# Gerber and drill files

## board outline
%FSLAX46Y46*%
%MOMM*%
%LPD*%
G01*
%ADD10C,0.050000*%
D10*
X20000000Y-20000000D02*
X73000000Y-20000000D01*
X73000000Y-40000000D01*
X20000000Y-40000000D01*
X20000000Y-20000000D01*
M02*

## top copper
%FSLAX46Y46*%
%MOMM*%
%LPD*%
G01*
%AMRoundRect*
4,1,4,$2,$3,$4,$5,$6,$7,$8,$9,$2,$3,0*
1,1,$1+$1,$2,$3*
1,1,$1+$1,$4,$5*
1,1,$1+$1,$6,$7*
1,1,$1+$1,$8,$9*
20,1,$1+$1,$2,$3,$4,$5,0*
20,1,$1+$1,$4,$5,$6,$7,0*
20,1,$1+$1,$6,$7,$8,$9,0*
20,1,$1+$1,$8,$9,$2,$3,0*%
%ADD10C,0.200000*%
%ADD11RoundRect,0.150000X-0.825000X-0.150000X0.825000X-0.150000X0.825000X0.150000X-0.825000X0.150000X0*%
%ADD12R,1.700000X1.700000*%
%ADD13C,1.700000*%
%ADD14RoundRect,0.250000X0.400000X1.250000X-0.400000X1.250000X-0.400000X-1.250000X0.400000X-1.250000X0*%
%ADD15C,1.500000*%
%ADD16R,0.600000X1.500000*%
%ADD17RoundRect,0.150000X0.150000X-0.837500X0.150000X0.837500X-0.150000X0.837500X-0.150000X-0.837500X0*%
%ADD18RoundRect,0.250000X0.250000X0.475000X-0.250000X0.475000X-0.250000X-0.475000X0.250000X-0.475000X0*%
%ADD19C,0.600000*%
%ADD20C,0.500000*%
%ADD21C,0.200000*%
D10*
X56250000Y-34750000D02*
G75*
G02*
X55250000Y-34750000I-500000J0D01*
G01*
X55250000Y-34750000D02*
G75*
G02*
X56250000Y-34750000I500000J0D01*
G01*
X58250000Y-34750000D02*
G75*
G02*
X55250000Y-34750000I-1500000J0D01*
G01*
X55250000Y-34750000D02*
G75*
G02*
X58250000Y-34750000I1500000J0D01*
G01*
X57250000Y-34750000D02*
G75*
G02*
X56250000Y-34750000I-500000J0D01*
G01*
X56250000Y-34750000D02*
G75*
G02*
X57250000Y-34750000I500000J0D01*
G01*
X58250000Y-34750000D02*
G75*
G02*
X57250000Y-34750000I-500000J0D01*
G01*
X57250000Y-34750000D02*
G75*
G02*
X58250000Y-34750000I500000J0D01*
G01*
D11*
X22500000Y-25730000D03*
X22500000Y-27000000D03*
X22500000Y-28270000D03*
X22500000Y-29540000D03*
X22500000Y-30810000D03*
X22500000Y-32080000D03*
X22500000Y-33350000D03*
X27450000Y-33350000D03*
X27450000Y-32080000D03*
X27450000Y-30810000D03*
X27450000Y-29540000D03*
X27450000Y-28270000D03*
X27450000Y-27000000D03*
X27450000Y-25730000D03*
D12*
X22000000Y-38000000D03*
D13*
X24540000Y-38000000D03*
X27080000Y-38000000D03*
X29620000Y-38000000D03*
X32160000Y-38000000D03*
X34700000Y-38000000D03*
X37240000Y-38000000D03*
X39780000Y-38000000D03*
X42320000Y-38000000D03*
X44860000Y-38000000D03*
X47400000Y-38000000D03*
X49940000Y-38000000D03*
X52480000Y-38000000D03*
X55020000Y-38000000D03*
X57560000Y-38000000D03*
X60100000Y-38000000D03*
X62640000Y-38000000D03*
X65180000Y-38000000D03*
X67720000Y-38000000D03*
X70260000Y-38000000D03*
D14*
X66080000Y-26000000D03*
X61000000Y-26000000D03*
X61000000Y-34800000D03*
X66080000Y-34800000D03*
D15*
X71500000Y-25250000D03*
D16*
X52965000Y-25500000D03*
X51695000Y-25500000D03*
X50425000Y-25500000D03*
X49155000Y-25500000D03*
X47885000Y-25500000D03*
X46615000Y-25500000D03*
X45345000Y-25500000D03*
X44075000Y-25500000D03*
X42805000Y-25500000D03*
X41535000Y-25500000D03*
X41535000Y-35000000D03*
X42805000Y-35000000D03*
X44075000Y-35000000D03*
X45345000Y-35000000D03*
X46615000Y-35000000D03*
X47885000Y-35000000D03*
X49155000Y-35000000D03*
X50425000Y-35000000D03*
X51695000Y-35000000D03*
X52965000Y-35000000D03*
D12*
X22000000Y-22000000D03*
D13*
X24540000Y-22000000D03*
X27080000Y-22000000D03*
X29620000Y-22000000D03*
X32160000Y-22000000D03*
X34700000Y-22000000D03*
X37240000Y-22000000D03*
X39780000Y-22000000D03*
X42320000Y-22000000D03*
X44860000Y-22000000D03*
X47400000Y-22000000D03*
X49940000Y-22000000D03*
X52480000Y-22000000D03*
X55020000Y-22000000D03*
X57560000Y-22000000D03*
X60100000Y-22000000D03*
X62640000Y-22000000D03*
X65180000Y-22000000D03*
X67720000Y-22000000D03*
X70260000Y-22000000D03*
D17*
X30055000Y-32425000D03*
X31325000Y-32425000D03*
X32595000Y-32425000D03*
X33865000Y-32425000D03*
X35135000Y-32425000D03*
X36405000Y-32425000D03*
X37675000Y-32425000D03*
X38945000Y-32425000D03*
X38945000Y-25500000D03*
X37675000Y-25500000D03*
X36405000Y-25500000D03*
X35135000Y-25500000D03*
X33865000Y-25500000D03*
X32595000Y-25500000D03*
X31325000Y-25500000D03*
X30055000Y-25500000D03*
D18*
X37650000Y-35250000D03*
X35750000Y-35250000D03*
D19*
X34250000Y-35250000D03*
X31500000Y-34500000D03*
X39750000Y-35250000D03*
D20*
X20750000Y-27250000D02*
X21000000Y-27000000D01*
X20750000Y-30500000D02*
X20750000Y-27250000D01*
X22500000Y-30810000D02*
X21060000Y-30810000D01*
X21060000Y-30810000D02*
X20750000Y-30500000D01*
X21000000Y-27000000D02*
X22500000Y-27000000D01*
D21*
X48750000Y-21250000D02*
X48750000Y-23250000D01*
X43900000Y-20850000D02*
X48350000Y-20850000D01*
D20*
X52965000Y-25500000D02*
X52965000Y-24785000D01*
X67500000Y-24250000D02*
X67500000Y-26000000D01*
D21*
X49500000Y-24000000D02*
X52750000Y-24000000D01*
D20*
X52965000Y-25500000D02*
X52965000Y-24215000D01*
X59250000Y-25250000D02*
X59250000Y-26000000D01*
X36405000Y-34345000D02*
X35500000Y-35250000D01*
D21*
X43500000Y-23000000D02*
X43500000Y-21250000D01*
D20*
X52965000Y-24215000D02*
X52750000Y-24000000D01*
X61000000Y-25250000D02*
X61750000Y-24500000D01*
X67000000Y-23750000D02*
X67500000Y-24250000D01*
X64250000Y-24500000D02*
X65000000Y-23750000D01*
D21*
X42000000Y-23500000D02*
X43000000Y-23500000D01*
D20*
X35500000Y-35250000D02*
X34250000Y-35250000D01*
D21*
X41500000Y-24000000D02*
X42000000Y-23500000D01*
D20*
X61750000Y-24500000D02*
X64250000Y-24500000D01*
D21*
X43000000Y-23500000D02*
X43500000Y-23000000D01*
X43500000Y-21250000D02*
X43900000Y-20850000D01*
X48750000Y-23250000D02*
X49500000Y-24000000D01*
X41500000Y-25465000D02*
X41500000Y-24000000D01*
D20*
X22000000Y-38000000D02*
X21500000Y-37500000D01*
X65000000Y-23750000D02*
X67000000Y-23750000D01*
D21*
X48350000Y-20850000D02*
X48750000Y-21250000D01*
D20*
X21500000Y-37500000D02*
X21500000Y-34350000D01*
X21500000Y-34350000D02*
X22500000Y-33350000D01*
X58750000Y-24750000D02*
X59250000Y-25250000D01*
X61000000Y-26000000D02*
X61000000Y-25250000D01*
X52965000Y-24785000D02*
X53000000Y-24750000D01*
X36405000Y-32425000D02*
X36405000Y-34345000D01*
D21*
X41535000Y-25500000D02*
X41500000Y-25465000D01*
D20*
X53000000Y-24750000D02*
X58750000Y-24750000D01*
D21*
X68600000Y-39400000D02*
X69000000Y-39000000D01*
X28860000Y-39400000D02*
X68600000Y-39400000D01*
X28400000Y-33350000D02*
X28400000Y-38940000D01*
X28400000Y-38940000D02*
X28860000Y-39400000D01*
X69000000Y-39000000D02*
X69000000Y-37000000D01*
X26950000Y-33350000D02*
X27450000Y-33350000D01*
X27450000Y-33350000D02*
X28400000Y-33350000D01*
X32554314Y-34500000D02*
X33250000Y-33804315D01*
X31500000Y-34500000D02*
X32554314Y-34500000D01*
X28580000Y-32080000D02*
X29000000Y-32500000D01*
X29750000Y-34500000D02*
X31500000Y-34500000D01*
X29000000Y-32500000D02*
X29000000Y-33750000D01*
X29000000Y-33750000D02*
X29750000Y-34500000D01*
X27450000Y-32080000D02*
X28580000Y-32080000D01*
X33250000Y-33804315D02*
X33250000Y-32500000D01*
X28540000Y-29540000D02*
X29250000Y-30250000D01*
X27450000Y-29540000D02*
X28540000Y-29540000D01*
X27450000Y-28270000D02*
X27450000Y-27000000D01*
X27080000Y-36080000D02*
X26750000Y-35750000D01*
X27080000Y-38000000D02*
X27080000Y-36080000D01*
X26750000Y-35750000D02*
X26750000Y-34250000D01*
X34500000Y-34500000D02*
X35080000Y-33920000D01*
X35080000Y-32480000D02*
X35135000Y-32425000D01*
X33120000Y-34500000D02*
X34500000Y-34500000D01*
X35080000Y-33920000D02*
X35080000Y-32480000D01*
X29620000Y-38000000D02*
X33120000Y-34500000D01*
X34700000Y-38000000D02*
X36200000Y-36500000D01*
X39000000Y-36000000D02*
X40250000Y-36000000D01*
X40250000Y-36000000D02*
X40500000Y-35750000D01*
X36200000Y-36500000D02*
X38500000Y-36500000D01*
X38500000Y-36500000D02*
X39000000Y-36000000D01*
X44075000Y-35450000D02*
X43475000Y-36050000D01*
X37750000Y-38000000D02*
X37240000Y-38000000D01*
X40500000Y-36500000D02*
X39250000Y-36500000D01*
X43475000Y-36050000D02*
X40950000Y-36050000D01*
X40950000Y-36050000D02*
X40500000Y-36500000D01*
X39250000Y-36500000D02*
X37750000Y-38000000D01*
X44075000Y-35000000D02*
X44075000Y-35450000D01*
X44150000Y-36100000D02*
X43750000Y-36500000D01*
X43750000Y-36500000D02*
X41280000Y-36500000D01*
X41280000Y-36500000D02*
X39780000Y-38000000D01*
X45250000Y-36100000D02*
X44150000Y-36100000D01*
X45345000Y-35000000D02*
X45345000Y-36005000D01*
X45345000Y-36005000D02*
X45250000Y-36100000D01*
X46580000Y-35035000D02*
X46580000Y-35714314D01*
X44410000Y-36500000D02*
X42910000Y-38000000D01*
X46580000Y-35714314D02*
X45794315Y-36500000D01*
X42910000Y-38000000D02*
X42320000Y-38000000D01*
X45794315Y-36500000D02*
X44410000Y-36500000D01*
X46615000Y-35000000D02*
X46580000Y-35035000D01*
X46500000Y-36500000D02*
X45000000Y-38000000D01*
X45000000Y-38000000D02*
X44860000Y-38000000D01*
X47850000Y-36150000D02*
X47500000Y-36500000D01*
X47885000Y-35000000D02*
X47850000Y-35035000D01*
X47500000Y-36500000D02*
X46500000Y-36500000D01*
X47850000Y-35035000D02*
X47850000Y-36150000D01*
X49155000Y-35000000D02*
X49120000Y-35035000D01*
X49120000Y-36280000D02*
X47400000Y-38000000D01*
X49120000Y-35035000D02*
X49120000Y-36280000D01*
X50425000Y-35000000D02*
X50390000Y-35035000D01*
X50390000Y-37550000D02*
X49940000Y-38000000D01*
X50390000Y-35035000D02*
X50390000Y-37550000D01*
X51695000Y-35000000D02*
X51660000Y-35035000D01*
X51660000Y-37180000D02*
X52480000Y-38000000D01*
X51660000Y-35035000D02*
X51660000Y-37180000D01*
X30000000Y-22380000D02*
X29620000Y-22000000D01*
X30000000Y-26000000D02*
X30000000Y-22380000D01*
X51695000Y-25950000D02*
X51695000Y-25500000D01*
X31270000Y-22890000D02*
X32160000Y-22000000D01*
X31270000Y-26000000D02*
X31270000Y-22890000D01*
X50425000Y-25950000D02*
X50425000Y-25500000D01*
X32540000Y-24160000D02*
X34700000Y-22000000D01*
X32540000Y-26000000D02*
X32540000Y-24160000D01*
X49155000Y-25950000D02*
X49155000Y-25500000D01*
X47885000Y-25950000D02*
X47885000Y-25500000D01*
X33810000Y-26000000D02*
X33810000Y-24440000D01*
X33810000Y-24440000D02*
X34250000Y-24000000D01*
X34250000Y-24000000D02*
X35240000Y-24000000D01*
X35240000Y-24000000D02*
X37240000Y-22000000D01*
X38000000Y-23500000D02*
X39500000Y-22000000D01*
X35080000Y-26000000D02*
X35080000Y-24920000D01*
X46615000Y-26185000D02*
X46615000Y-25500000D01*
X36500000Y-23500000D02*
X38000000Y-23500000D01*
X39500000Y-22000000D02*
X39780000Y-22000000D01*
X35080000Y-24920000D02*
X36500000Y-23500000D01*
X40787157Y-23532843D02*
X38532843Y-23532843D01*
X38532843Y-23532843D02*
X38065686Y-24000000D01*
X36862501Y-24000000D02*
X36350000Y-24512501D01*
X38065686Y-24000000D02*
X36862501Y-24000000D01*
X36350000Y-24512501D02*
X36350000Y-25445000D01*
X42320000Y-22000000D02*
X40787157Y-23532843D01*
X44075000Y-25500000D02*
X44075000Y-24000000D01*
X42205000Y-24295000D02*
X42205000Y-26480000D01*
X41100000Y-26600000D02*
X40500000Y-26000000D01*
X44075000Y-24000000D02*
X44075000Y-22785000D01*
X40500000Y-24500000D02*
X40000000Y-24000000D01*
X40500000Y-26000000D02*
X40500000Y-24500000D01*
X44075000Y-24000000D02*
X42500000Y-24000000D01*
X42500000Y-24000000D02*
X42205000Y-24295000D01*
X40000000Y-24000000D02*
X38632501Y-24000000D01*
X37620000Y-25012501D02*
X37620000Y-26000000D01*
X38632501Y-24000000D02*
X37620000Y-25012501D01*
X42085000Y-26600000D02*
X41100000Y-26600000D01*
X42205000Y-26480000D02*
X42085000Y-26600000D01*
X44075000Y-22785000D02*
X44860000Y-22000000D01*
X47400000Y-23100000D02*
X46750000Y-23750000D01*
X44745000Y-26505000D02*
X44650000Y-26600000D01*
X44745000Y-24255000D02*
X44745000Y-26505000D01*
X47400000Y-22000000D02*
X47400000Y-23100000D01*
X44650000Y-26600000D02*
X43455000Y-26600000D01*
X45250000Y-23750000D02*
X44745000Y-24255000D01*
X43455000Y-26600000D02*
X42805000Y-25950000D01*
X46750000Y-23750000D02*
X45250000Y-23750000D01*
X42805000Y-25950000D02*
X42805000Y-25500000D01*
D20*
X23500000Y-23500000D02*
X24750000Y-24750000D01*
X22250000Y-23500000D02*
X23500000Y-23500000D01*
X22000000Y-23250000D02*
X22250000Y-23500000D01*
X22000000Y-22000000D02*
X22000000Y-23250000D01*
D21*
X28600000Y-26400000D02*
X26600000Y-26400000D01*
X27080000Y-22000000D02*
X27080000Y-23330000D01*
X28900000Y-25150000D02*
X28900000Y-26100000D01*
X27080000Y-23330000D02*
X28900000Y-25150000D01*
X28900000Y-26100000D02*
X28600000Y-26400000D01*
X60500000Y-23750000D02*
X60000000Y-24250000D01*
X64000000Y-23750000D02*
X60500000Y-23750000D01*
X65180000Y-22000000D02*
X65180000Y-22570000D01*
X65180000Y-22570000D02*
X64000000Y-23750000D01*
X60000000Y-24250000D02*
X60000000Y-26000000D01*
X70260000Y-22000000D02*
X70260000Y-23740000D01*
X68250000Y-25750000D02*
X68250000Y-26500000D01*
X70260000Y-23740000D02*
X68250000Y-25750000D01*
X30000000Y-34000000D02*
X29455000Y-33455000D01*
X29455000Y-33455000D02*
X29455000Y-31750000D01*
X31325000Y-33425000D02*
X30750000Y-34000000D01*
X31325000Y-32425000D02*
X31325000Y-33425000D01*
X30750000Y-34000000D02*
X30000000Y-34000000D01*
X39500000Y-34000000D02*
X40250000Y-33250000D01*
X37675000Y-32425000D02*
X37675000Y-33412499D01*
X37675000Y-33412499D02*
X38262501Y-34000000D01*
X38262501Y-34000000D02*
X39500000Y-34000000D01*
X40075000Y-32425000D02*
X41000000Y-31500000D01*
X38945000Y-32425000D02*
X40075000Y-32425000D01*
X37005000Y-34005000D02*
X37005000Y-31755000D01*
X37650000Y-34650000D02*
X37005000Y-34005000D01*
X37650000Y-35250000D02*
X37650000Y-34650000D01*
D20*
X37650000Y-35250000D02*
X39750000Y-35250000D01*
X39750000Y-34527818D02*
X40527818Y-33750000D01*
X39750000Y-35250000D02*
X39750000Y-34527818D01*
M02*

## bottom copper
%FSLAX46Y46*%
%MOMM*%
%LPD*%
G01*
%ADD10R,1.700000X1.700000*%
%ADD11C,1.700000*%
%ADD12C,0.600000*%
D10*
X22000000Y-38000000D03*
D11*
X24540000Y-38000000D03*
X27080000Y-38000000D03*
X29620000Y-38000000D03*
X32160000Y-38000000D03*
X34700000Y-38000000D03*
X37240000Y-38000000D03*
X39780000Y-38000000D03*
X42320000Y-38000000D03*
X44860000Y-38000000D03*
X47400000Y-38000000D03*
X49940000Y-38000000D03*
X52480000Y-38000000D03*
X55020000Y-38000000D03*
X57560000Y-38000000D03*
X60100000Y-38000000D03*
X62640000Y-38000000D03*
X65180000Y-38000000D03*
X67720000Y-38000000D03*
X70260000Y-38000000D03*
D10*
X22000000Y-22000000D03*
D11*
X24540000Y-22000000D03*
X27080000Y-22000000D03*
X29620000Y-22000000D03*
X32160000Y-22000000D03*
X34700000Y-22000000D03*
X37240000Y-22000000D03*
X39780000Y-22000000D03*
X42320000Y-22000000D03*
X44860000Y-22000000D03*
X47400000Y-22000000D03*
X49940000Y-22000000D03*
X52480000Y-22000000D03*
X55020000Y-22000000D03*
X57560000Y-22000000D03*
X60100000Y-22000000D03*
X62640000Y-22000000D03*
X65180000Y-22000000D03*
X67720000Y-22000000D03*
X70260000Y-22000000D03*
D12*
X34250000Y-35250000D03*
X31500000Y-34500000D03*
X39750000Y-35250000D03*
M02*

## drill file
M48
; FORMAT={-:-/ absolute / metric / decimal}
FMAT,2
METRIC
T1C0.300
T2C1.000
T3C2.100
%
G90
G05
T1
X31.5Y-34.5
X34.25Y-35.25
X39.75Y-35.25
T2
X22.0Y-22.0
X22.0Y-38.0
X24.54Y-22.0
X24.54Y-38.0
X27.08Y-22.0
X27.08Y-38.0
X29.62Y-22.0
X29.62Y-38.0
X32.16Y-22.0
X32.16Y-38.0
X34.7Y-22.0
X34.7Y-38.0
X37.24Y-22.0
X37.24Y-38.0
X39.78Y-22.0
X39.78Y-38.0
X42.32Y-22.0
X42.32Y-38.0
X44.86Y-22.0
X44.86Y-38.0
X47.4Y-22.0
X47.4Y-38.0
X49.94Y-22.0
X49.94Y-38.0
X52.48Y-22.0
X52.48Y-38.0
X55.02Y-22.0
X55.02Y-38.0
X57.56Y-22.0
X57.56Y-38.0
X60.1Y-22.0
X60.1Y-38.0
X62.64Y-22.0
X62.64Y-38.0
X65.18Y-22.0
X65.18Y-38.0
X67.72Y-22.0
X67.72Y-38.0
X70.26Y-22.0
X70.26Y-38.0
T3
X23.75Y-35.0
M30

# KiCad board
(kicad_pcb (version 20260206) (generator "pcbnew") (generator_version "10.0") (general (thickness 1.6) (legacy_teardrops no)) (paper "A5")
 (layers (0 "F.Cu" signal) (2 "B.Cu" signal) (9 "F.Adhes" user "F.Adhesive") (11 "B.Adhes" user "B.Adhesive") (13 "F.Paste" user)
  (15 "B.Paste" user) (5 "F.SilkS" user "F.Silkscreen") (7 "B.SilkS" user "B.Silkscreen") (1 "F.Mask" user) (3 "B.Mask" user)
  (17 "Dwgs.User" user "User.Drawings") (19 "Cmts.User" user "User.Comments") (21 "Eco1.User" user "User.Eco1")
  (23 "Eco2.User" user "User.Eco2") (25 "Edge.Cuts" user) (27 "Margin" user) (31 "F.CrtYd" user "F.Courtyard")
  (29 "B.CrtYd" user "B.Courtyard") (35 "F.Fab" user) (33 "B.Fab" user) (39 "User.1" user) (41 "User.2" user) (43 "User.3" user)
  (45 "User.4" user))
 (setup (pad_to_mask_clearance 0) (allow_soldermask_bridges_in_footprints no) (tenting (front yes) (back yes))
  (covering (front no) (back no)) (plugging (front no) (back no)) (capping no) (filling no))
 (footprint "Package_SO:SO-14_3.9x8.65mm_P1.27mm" (layer "F.Cu") (at 24.975 29.54)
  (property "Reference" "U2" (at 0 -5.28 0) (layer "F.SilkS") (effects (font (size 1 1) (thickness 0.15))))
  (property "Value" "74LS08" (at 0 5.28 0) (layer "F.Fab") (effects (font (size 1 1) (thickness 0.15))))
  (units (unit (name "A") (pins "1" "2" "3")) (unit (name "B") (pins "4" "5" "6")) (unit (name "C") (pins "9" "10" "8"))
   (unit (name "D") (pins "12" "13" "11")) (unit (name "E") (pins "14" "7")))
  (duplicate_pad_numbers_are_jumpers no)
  (pad "1" smd roundrect (at -2.475 -3.81) (size 1.95 0.6) (layers "F.Cu" "F.Mask" "F.Paste") (roundrect_rratio 0.25)
   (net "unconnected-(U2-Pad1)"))
  (pad "2" smd roundrect (at -2.475 -2.54) (size 1.95 0.6) (layers "F.Cu" "F.Mask" "F.Paste") (roundrect_rratio 0.25) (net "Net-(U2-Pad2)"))
  (pad "3" smd roundrect (at -2.475 -1.27) (size 1.95 0.6) (layers "F.Cu" "F.Mask" "F.Paste") (roundrect_rratio 0.25)
   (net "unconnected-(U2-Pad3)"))
  (pad "4" smd roundrect (at -2.475 0) (size 1.95 0.6) (layers "F.Cu" "F.Mask" "F.Paste") (roundrect_rratio 0.25)
   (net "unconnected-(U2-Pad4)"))
  (pad "5" smd roundrect (at -2.475 1.27) (size 1.95 0.6) (layers "F.Cu" "F.Mask" "F.Paste") (roundrect_rratio 0.25) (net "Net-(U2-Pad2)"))
  (pad "6" smd roundrect (at -2.475 2.54) (size 1.95 0.6) (layers "F.Cu" "F.Mask" "F.Paste") (roundrect_rratio 0.25)
   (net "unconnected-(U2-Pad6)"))
  (pad "7" smd roundrect (at -2.475 3.81) (size 1.95 0.6) (layers "F.Cu" "F.Mask" "F.Paste") (roundrect_rratio 0.25) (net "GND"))
  (pad "8" smd roundrect (at 2.475 3.81) (size 1.95 0.6) (layers "F.Cu" "F.Mask" "F.Paste") (roundrect_rratio 0.25)
   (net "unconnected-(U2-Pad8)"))
  (pad "9" smd roundrect (at 2.475 2.54) (size 1.95 0.6) (layers "F.Cu" "F.Mask" "F.Paste") (roundrect_rratio 0.25)
   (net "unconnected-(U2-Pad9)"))
  (pad "10" smd roundrect (at 2.475 1.27) (size 1.95 0.6) (layers "F.Cu" "F.Mask" "F.Paste") (roundrect_rratio 0.25)
   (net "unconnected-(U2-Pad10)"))
  (pad "11" smd roundrect (at 2.475 0) (size 1.95 0.6) (layers "F.Cu" "F.Mask" "F.Paste") (roundrect_rratio 0.25)
   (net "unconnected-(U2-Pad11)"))
  (pad "12" smd roundrect (at 2.475 -1.27) (size 1.95 0.6) (layers "F.Cu" "F.Mask" "F.Paste") (roundrect_rratio 0.25) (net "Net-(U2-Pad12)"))
  (pad "13" smd roundrect (at 2.475 -2.54) (size 1.95 0.6) (layers "F.Cu" "F.Mask" "F.Paste") (roundrect_rratio 0.25) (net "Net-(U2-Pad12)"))
  (pad "14" smd roundrect (at 2.475 -3.81) (size 1.95 0.6) (layers "F.Cu" "F.Mask" "F.Paste") (roundrect_rratio 0.25)
   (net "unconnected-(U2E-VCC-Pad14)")))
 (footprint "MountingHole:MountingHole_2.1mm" (layer "F.Cu") (at 23.75 35)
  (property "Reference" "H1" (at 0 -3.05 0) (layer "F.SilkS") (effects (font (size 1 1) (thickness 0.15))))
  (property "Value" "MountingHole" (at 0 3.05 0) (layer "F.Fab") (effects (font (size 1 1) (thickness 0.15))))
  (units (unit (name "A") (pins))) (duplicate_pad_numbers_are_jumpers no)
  (pad "" np_thru_hole circle (at 0 0) (size 2.1 2.1) (drill 2.1) (layers "*.Cu" "*.Mask")))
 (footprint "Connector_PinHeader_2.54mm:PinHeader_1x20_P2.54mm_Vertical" (layer "F.Cu") (at 22 38 90)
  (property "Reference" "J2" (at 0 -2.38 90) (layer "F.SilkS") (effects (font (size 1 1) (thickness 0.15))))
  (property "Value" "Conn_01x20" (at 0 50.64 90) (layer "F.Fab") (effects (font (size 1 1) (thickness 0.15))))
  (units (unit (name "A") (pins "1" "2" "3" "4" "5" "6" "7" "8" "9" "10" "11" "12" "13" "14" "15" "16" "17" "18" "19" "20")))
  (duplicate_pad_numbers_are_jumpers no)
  (pad "1" thru_hole rect (at 0 0 90) (size 1.7 1.7) (drill 1) (layers "*.Cu" "*.Mask") (remove_unused_layers no) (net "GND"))
  (pad "2" thru_hole circle (at 0 2.54 90) (size 1.7 1.7) (drill 1) (layers "*.Cu" "*.Mask") (remove_unused_layers no)
   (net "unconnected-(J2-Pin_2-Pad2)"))
  (pad "3" thru_hole circle (at 0 5.08 90) (size 1.7 1.7) (drill 1) (layers "*.Cu" "*.Mask") (remove_unused_layers no)
   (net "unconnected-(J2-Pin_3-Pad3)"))
  (pad "4" thru_hole circle (at 0 7.62 90) (size 1.7 1.7) (drill 1) (layers "*.Cu" "*.Mask") (remove_unused_layers no) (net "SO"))
  (pad "5" thru_hole circle (at 0 10.16 90) (size 1.7 1.7) (drill 1) (layers "*.Cu" "*.Mask") (remove_unused_layers no)
   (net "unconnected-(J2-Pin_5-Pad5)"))
  (pad "6" thru_hole circle (at 0 12.7 90) (size 1.7 1.7) (drill 1) (layers "*.Cu" "*.Mask") (remove_unused_layers no)
   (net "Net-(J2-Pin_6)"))
  (pad "7" thru_hole circle (at 0 15.24 90) (size 1.7 1.7) (drill 1) (layers "*.Cu" "*.Mask") (remove_unused_layers no)
   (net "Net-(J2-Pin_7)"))
  (pad "8" thru_hole circle (at 0 17.78 90) (size 1.7 1.7) (drill 1) (layers "*.Cu" "*.Mask") (remove_unused_layers no)
   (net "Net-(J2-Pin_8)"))
  (pad "9" thru_hole circle (at 0 20.32 90) (size 1.7 1.7) (drill 1) (layers "*.Cu" "*.Mask") (remove_unused_layers no)
   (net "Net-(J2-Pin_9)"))
  (pad "10" thru_hole circle (at 0 22.86 90) (size 1.7 1.7) (drill 1) (layers "*.Cu" "*.Mask") (remove_unused_layers no)
   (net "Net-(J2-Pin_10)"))
  (pad "11" thru_hole circle (at 0 25.4 90) (size 1.7 1.7) (drill 1) (layers "*.Cu" "*.Mask") (remove_unused_layers no)
   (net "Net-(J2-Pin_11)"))
  (pad "12" thru_hole circle (at 0 27.94 90) (size 1.7 1.7) (drill 1) (layers "*.Cu" "*.Mask") (remove_unused_layers no)
   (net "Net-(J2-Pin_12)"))
  (pad "13" thru_hole circle (at 0 30.48 90) (size 1.7 1.7) (drill 1) (layers "*.Cu" "*.Mask") (remove_unused_layers no)
   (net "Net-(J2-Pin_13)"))
  (pad "14" thru_hole circle (at 0 33.02 90) (size 1.7 1.7) (drill 1) (layers "*.Cu" "*.Mask") (remove_unused_layers no)
   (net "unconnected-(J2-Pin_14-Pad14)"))
  (pad "15" thru_hole circle (at 0 35.56 90) (size 1.7 1.7) (drill 1) (layers "*.Cu" "*.Mask") (remove_unused_layers no)
   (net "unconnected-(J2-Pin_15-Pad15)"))
  (pad "16" thru_hole circle (at 0 38.1 90) (size 1.7 1.7) (drill 1) (layers "*.Cu" "*.Mask") (remove_unused_layers no)
   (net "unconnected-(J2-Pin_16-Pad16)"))
  (pad "17" thru_hole circle (at 0 40.64 90) (size 1.7 1.7) (drill 1) (layers "*.Cu" "*.Mask") (remove_unused_layers no)
   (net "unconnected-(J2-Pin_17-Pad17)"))
  (pad "18" thru_hole circle (at 0 43.18 90) (size 1.7 1.7) (drill 1) (layers "*.Cu" "*.Mask") (remove_unused_layers no)
   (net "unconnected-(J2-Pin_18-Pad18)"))
  (pad "19" thru_hole circle (at 0 45.72 90) (size 1.7 1.7) (drill 1) (layers "*.Cu" "*.Mask") (remove_unused_layers no)
   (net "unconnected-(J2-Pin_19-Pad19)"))
  (pad "20" thru_hole circle (at 0 48.26 90) (size 1.7 1.7) (drill 1) (layers "*.Cu" "*.Mask") (remove_unused_layers no)
   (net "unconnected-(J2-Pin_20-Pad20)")))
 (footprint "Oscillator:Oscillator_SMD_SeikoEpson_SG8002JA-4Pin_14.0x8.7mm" (layer "F.Cu") (at 63.54 30.4 180)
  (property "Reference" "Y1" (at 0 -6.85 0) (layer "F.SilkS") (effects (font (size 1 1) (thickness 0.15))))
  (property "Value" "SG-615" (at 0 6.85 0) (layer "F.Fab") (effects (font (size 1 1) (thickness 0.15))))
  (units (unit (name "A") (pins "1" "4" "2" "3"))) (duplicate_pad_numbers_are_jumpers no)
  (pad "1" smd roundrect (at -2.54 4.4 180) (size 1.3 3) (layers "F.Cu" "F.Mask" "F.Paste") (roundrect_rratio 0.192308)
   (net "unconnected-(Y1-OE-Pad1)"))
  (pad "2" smd roundrect (at 2.54 4.4 180) (size 1.3 3) (layers "F.Cu" "F.Mask" "F.Paste") (roundrect_rratio 0.192308) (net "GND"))
  (pad "3" smd roundrect (at 2.54 -4.4 180) (size 1.3 3) (layers "F.Cu" "F.Mask" "F.Paste") (roundrect_rratio 0.192308)
   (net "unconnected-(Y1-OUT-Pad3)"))
  (pad "4" smd roundrect (at -2.54 -4.4 180) (size 1.3 3) (layers "F.Cu" "F.Mask" "F.Paste") (roundrect_rratio 0.192308)
   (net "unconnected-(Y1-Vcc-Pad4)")))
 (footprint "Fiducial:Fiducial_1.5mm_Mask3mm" (layer "F.Cu") (at 71.5 25.25)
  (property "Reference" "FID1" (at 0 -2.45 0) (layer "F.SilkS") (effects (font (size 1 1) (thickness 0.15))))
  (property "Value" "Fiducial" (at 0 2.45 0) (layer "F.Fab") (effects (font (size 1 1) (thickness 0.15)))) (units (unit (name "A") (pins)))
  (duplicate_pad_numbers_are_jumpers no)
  (pad "" smd circle (at 0 0) (size 1.5 1.5) (layers "F.Cu" "F.Mask") (solder_mask_margin 0.75) (clearance 0.85)))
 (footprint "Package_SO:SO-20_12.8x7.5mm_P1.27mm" (layer "F.Cu") (at 47.25 30.25 -90)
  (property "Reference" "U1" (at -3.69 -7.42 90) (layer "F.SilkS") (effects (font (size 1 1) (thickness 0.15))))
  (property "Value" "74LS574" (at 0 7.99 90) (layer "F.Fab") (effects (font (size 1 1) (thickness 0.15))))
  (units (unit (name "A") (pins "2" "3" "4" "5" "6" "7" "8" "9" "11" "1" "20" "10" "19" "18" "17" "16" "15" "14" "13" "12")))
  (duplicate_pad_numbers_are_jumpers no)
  (pad "1" smd rect (at -4.75 -5.715 270) (size 1.5 0.6) (layers "F.Cu" "F.Mask" "F.Paste") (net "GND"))
  (pad "2" smd rect (at -4.75 -4.445 270) (size 1.5 0.6) (layers "F.Cu" "F.Mask" "F.Paste") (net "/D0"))
  (pad "3" smd rect (at -4.75 -3.175 270) (size 1.5 0.6) (layers "F.Cu" "F.Mask" "F.Paste") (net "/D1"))
  (pad "4" smd rect (at -4.75 -1.905 270) (size 1.5 0.6) (layers "F.Cu" "F.Mask" "F.Paste") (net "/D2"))
  (pad "5" smd rect (at -4.75 -0.635 270) (size 1.5 0.6) (layers "F.Cu" "F.Mask" "F.Paste") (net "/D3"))
  (pad "6" smd rect (at -4.75 0.635 270) (size 1.5 0.6) (layers "F.Cu" "F.Mask" "F.Paste") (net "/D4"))
  (pad "7" smd rect (at -4.75 1.905 270) (size 1.5 0.6) (layers "F.Cu" "F.Mask" "F.Paste") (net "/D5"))
  (pad "8" smd rect (at -4.75 3.175 270) (size 1.5 0.6) (layers "F.Cu" "F.Mask" "F.Paste") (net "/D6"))
  (pad "9" smd rect (at -4.75 4.445 270) (size 1.5 0.6) (layers "F.Cu" "F.Mask" "F.Paste") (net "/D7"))
  (pad "10" smd rect (at -4.75 5.715 270) (size 1.5 0.6) (layers "F.Cu" "F.Mask" "F.Paste") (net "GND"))
  (pad "11" smd rect (at 4.75 5.715 270) (size 1.5 0.6) (layers "F.Cu" "F.Mask" "F.Paste") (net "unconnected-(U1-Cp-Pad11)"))
  (pad "12" smd rect (at 4.75 4.445 270) (size 1.5 0.6) (layers "F.Cu" "F.Mask" "F.Paste") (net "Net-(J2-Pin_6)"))
  (pad "13" smd rect (at 4.75 3.175 270) (size 1.5 0.6) (layers "F.Cu" "F.Mask" "F.Paste") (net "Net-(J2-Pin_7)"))
  (pad "14" smd rect (at 4.75 1.905 270) (size 1.5 0.6) (layers "F.Cu" "F.Mask" "F.Paste") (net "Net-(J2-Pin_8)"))
  (pad "15" smd rect (at 4.75 0.635 270) (size 1.5 0.6) (layers "F.Cu" "F.Mask" "F.Paste") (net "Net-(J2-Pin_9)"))
  (pad "16" smd rect (at 4.75 -0.635 270) (size 1.5 0.6) (layers "F.Cu" "F.Mask" "F.Paste") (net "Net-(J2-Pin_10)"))
  (pad "17" smd rect (at 4.75 -1.905 270) (size 1.5 0.6) (layers "F.Cu" "F.Mask" "F.Paste") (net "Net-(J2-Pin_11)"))
  (pad "18" smd rect (at 4.75 -3.175 270) (size 1.5 0.6) (layers "F.Cu" "F.Mask" "F.Paste") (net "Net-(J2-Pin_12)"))
  (pad "19" smd rect (at 4.75 -4.445 270) (size 1.5 0.6) (layers "F.Cu" "F.Mask" "F.Paste") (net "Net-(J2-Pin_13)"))
  (pad "20" smd rect (at 4.75 -5.715 270) (size 1.5 0.6) (layers "F.Cu" "F.Mask" "F.Paste") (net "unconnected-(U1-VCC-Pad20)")))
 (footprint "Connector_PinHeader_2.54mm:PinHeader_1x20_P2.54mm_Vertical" (layer "F.Cu") (at 22 22 90)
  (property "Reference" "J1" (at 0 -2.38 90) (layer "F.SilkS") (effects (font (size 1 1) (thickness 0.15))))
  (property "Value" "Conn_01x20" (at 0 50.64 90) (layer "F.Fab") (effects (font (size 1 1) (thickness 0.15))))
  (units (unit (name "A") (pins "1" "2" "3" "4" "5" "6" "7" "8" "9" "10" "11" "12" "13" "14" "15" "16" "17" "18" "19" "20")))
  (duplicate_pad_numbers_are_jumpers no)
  (pad "1" thru_hole rect (at 0 0 90) (size 1.7 1.7) (drill 1) (layers "*.Cu" "*.Mask") (remove_unused_layers no) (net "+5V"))
  (pad "2" thru_hole circle (at 0 2.54 90) (size 1.7 1.7) (drill 1) (layers "*.Cu" "*.Mask") (remove_unused_layers no)
   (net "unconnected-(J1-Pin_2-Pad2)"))
  (pad "3" thru_hole circle (at 0 5.08 90) (size 1.7 1.7) (drill 1) (layers "*.Cu" "*.Mask") (remove_unused_layers no)
   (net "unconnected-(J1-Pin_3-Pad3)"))
  (pad "4" thru_hole circle (at 0 7.62 90) (size 1.7 1.7) (drill 1) (layers "*.Cu" "*.Mask") (remove_unused_layers no) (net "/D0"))
  (pad "5" thru_hole circle (at 0 10.16 90) (size 1.7 1.7) (drill 1) (layers "*.Cu" "*.Mask") (remove_unused_layers no) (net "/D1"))
  (pad "6" thru_hole circle (at 0 12.7 90) (size 1.7 1.7) (drill 1) (layers "*.Cu" "*.Mask") (remove_unused_layers no) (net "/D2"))
  (pad "7" thru_hole circle (at 0 15.24 90) (size 1.7 1.7) (drill 1) (layers "*.Cu" "*.Mask") (remove_unused_layers no) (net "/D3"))
  (pad "8" thru_hole circle (at 0 17.78 90) (size 1.7 1.7) (drill 1) (layers "*.Cu" "*.Mask") (remove_unused_layers no) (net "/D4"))
  (pad "9" thru_hole circle (at 0 20.32 90) (size 1.7 1.7) (drill 1) (layers "*.Cu" "*.Mask") (remove_unused_layers no) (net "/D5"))
  (pad "10" thru_hole circle (at 0 22.86 90) (size 1.7 1.7) (drill 1) (layers "*.Cu" "*.Mask") (remove_unused_layers no) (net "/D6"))
  (pad "11" thru_hole circle (at 0 25.4 90) (size 1.7 1.7) (drill 1) (layers "*.Cu" "*.Mask") (remove_unused_layers no) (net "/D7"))
  (pad "12" thru_hole circle (at 0 27.94 90) (size 1.7 1.7) (drill 1) (layers "*.Cu" "*.Mask") (remove_unused_layers no)
   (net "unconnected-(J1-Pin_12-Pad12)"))
  (pad "13" thru_hole circle (at 0 30.48 90) (size 1.7 1.7) (drill 1) (layers "*.Cu" "*.Mask") (remove_unused_layers no) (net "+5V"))
  (pad "14" thru_hole circle (at 0 33.02 90) (size 1.7 1.7) (drill 1) (layers "*.Cu" "*.Mask") (remove_unused_layers no)
   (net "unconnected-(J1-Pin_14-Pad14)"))
  (pad "15" thru_hole circle (at 0 35.56 90) (size 1.7 1.7) (drill 1) (layers "*.Cu" "*.Mask") (remove_unused_layers no)
   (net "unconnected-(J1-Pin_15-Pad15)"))
  (pad "16" thru_hole circle (at 0 38.1 90) (size 1.7 1.7) (drill 1) (layers "*.Cu" "*.Mask") (remove_unused_layers no) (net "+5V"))
  (pad "17" thru_hole circle (at 0 40.64 90) (size 1.7 1.7) (drill 1) (layers "*.Cu" "*.Mask") (remove_unused_layers no)
   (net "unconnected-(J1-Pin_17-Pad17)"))
  (pad "18" thru_hole circle (at 0 43.18 90) (size 1.7 1.7) (drill 1) (layers "*.Cu" "*.Mask") (remove_unused_layers no)
   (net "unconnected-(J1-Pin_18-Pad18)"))
  (pad "19" thru_hole circle (at 0 45.72 90) (size 1.7 1.7) (drill 1) (layers "*.Cu" "*.Mask") (remove_unused_layers no)
   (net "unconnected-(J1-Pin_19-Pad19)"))
  (pad "20" thru_hole circle (at 0 48.26 90) (size 1.7 1.7) (drill 1) (layers "*.Cu" "*.Mask") (remove_unused_layers no)
   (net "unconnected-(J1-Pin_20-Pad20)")))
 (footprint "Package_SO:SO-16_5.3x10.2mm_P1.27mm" (layer "F.Cu") (at 34.5 28.9625 90)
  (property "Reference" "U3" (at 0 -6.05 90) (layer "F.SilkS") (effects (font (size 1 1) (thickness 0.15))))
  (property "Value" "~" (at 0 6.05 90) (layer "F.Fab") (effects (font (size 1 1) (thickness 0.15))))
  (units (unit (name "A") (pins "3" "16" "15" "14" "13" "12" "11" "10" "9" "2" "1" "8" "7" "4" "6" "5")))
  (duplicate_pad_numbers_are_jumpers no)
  (pad "1" smd roundrect (at -3.4625 -4.445 90) (size 1.975 0.6) (layers "F.Cu" "F.Mask" "F.Paste") (roundrect_rratio 0.25)
   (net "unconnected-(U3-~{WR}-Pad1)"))
  (pad "2" smd roundrect (at -3.4625 -3.175 90) (size 1.975 0.6) (layers "F.Cu" "F.Mask" "F.Paste") (roundrect_rratio 0.25)
   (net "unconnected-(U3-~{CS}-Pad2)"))
  (pad "3" smd roundrect (at -3.4625 -1.905 90) (size 1.975 0.6) (layers "F.Cu" "F.Mask" "F.Paste") (roundrect_rratio 0.25)
   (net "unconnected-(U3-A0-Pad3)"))
  (pad "4" smd roundrect (at -3.4625 -0.635 90) (size 1.975 0.6) (layers "F.Cu" "F.Mask" "F.Paste") (roundrect_rratio 0.25)
   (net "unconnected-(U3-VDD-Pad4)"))
  (pad "5" smd roundrect (at -3.4625 0.635 90) (size 1.975 0.6) (layers "F.Cu" "F.Mask" "F.Paste") (roundrect_rratio 0.25) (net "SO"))
  (pad "6" smd roundrect (at -3.4625 1.905 90) (size 1.975 0.6) (layers "F.Cu" "F.Mask" "F.Paste") (roundrect_rratio 0.25) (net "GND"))
  (pad "7" smd roundrect (at -3.4625 3.175 90) (size 1.975 0.6) (layers "F.Cu" "F.Mask" "F.Paste") (roundrect_rratio 0.25)
   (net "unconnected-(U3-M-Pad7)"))
  (pad "8" smd roundrect (at -3.4625 4.445 90) (size 1.975 0.6) (layers "F.Cu" "F.Mask" "F.Paste") (roundrect_rratio 0.25)
   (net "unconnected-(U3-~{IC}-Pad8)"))
  (pad "9" smd roundrect (at 3.4625 4.445 90) (size 1.975 0.6) (layers "F.Cu" "F.Mask" "F.Paste") (roundrect_rratio 0.25) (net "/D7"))
  (pad "10" smd roundrect (at 3.4625 3.175 90) (size 1.975 0.6) (layers "F.Cu" "F.Mask" "F.Paste") (roundrect_rratio 0.25) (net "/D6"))
  (pad "11" smd roundrect (at 3.4625 1.905 90) (size 1.975 0.6) (layers "F.Cu" "F.Mask" "F.Paste") (roundrect_rratio 0.25) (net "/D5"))
  (pad "12" smd roundrect (at 3.4625 0.635 90) (size 1.975 0.6) (layers "F.Cu" "F.Mask" "F.Paste") (roundrect_rratio 0.25) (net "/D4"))
  (pad "13" smd roundrect (at 3.4625 -0.635 90) (size 1.975 0.6) (layers "F.Cu" "F.Mask" "F.Paste") (roundrect_rratio 0.25) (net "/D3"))
  (pad "14" smd roundrect (at 3.4625 -1.905 90) (size 1.975 0.6) (layers "F.Cu" "F.Mask" "F.Paste") (roundrect_rratio 0.25) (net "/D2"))
  (pad "15" smd roundrect (at 3.4625 -3.175 90) (size 1.975 0.6) (layers "F.Cu" "F.Mask" "F.Paste") (roundrect_rratio 0.25) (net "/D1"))
  (pad "16" smd roundrect (at 3.4625 -4.445 90) (size 1.975 0.6) (layers "F.Cu" "F.Mask" "F.Paste") (roundrect_rratio 0.25) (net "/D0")))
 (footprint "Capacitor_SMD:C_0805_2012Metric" (layer "F.Cu") (at 36.7 35.25 180)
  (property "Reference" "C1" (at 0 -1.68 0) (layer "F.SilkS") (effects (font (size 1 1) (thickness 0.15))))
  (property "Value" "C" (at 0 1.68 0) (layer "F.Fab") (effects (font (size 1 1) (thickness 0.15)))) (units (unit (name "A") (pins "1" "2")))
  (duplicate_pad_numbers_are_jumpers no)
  (pad "1" smd roundrect (at -0.95 0 180) (size 1 1.45) (layers "F.Cu" "F.Mask" "F.Paste") (roundrect_rratio 0.25)
   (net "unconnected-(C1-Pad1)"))
  (pad "2" smd roundrect (at 0.95 0 180) (size 1 1.45) (layers "F.Cu" "F.Mask" "F.Paste") (roundrect_rratio 0.25) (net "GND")))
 (gr_circle (center 55.75 34.75) (end 56.25 34.75) (stroke (width 0.2) (type default)) (fill no) (layer "F.Cu"))
 (gr_circle (center 56.75 34.75) (end 55.25 34.75) (stroke (width 0.2) (type default)) (fill no) (layer "F.Cu"))
 (gr_circle (center 56.75 34.75) (end 57.25 34.75) (stroke (width 0.2) (type default)) (fill no) (layer "F.Cu"))
 (gr_circle (center 57.75 34.75) (end 58.25 34.75) (stroke (width 0.2) (type default)) (fill no) (layer "F.Cu"))
 (gr_rect (start 20 20) (end 73 40) (stroke (width 0.05) (type default)) (fill no) (layer "Edge.Cuts"))
 (segment (start 20.75 27.25) (end 21 27) (width 0.5) (layer "F.Cu") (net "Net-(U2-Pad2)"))
 (segment (start 20.75 30.5) (end 20.75 27.25) (width 0.5) (layer "F.Cu") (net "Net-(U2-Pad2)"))
 (segment (start 22.5 30.81) (end 21.06 30.81) (width 0.5) (layer "F.Cu") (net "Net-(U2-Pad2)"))
 (segment (start 21.06 30.81) (end 20.75 30.5) (width 0.5) (layer "F.Cu") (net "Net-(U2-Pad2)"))
 (segment (start 21 27) (end 22.5 27) (width 0.5) (layer "F.Cu") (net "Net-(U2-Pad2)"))
 (segment (start 48.75 21.25) (end 48.75 23.25) (width 0.2) (layer "F.Cu") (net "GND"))
 (segment (start 43.9 20.85) (end 48.35 20.85) (width 0.2) (layer "F.Cu") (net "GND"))
 (segment (start 52.965 25.5) (end 52.965 24.785) (width 0.5) (layer "F.Cu") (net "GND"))
 (segment (start 67.5 24.25) (end 67.5 26) (width 0.5) (layer "F.Cu") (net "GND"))
 (segment (start 49.5 24) (end 52.75 24) (width 0.2) (layer "F.Cu") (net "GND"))
 (segment (start 52.965 25.5) (end 52.965 24.215) (width 0.5) (layer "F.Cu") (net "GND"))
 (segment (start 59.25 25.25) (end 59.25 26) (width 0.5) (layer "F.Cu") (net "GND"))
 (segment (start 36.405 34.345) (end 35.5 35.25) (width 0.5) (layer "F.Cu") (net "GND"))
 (segment (start 43.5 23) (end 43.5 21.25) (width 0.2) (layer "F.Cu") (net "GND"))
 (segment (start 52.965 24.215) (end 52.75 24) (width 0.5) (layer "F.Cu") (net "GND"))
 (segment (start 61 25.25) (end 61.75 24.5) (width 0.5) (layer "F.Cu") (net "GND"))
 (segment (start 67 23.75) (end 67.5 24.25) (width 0.5) (layer "F.Cu") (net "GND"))
 (segment (start 64.25 24.5) (end 65 23.75) (width 0.5) (layer "F.Cu") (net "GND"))
 (segment (start 42 23.5) (end 43 23.5) (width 0.2) (layer "F.Cu") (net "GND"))
 (segment (start 35.5 35.25) (end 34.25 35.25) (width 0.5) (layer "F.Cu") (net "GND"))
 (segment (start 41.5 24) (end 42 23.5) (width 0.2) (layer "F.Cu") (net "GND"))
 (segment (start 61.75 24.5) (end 64.25 24.5) (width 0.5) (layer "F.Cu") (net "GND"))
 (segment (start 43 23.5) (end 43.5 23) (width 0.2) (layer "F.Cu") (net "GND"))
 (segment (start 43.5 21.25) (end 43.9 20.85) (width 0.2) (layer "F.Cu") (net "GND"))
 (segment (start 48.75 23.25) (end 49.5 24) (width 0.2) (layer "F.Cu") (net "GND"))
 (segment (start 41.5 25.465) (end 41.5 24) (width 0.2) (layer "F.Cu") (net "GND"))
 (segment (start 22 38) (end 21.5 37.5) (width 0.5) (layer "F.Cu") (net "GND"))
 (segment (start 65 23.75) (end 67 23.75) (width 0.5) (layer "F.Cu") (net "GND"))
 (segment (start 48.35 20.85) (end 48.75 21.25) (width 0.2) (layer "F.Cu") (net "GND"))
 (segment (start 21.5 37.5) (end 21.5 34.35) (width 0.5) (layer "F.Cu") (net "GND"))
 (segment (start 21.5 34.35) (end 22.5 33.35) (width 0.5) (layer "F.Cu") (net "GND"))
 (segment (start 58.75 24.75) (end 59.25 25.25) (width 0.5) (layer "F.Cu") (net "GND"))
 (segment (start 61 26) (end 61 25.25) (width 0.5) (layer "F.Cu") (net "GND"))
 (segment (start 52.965 24.785) (end 53 24.75) (width 0.5) (layer "F.Cu") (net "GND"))
 (segment (start 36.405 32.425) (end 36.405 34.345) (width 0.5) (layer "F.Cu") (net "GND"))
 (segment (start 41.535 25.5) (end 41.5 25.465) (width 0.2) (layer "F.Cu") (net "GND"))
 (segment (start 53 24.75) (end 58.75 24.75) (width 0.5) (layer "F.Cu") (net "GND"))
 (via (at 34.25 35.25) (size 0.6) (drill 0.3) (layers "F.Cu" "B.Cu") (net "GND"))
 (segment (start 68.6 39.4) (end 69 39) (width 0.2) (layer "F.Cu") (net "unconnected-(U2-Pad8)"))
 (segment (start 28.86 39.4) (end 68.6 39.4) (width 0.2) (layer "F.Cu") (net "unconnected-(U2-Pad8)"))
 (segment (start 28.4 33.35) (end 28.4 38.94) (width 0.2) (layer "F.Cu") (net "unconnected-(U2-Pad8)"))
 (segment (start 28.4 38.94) (end 28.86 39.4) (width 0.2) (layer "F.Cu") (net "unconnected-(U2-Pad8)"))
 (segment (start 69 39) (end 69 37) (width 0.2) (layer "F.Cu") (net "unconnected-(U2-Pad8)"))
 (segment (start 26.95 33.35) (end 27.45 33.35) (width 0.2) (layer "F.Cu") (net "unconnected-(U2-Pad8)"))
 (segment (start 27.45 33.35) (end 28.4 33.35) (width 0.2) (layer "F.Cu") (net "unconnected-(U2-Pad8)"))
 (segment (start 32.554314 34.5) (end 33.25 33.804315) (width 0.2) (layer "F.Cu") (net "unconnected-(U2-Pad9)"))
 (segment (start 31.5 34.5) (end 32.554314 34.5) (width 0.2) (layer "F.Cu") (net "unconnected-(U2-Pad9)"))
 (segment (start 28.58 32.08) (end 29 32.5) (width 0.2) (layer "F.Cu") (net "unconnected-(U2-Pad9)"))
 (segment (start 29.75 34.5) (end 31.5 34.5) (width 0.2) (layer "F.Cu") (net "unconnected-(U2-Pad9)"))
 (segment (start 29 32.5) (end 29 33.75) (width 0.2) (layer "F.Cu") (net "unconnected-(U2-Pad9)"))
 (segment (start 29 33.75) (end 29.75 34.5) (width 0.2) (layer "F.Cu") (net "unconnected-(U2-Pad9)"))
 (segment (start 27.45 32.08) (end 28.58 32.08) (width 0.2) (layer "F.Cu") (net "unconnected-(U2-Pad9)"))
 (segment (start 33.25 33.804315) (end 33.25 32.5) (width 0.2) (layer "F.Cu") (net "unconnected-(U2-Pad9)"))
 (via (at 31.5 34.5) (size 0.6) (drill 0.3) (layers "F.Cu" "B.Cu") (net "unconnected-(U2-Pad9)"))
 (segment (start 28.54 29.54) (end 29.25 30.25) (width 0.2) (layer "F.Cu") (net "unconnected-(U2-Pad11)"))
 (segment (start 27.45 29.54) (end 28.54 29.54) (width 0.2) (layer "F.Cu") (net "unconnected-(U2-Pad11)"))
 (segment (start 27.45 28.27) (end 27.45 27) (width 0.2) (layer "F.Cu") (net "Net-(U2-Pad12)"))
 (segment (start 27.08 36.08) (end 26.75 35.75) (width 0.2) (layer "F.Cu") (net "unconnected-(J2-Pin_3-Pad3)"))
 (segment (start 27.08 38) (end 27.08 36.08) (width 0.2) (layer "F.Cu") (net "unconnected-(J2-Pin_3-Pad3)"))
 (segment (start 26.75 35.75) (end 26.75 34.25) (width 0.2) (layer "F.Cu") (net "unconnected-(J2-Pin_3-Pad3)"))
 (segment (start 34.5 34.5) (end 35.08 33.92) (width 0.2) (layer "F.Cu") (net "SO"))
 (segment (start 35.08 32.48) (end 35.135 32.425) (width 0.2) (layer "F.Cu") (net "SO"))
 (segment (start 33.12 34.5) (end 34.5 34.5) (width 0.2) (layer "F.Cu") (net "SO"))
 (segment (start 35.08 33.92) (end 35.08 32.48) (width 0.2) (layer "F.Cu") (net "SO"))
 (segment (start 29.62 38) (end 33.12 34.5) (width 0.2) (layer "F.Cu") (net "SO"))
 (segment (start 34.7 38) (end 36.2 36.5) (width 0.2) (layer "F.Cu") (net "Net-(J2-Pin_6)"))
 (segment (start 39 36) (end 40.25 36) (width 0.2) (layer "F.Cu") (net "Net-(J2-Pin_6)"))
 (segment (start 40.25 36) (end 40.5 35.75) (width 0.2) (layer "F.Cu") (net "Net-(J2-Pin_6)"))
 (segment (start 36.2 36.5) (end 38.5 36.5) (width 0.2) (layer "F.Cu") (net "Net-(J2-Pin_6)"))
 (segment (start 38.5 36.5) (end 39 36) (width 0.2) (layer "F.Cu") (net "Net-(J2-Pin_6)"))
 (segment (start 44.075 35.45) (end 43.475 36.05) (width 0.2) (layer "F.Cu") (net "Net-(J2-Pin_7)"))
 (segment (start 37.75 38) (end 37.24 38) (width 0.2) (layer "F.Cu") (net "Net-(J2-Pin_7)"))
 (segment (start 40.5 36.5) (end 39.25 36.5) (width 0.2) (layer "F.Cu") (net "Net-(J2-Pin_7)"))
 (segment (start 43.475 36.05) (end 40.95 36.05) (width 0.2) (layer "F.Cu") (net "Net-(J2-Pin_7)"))
 (segment (start 40.95 36.05) (end 40.5 36.5) (width 0.2) (layer "F.Cu") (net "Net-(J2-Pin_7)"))
 (segment (start 39.25 36.5) (end 37.75 38) (width 0.2) (layer "F.Cu") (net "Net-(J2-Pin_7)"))
 (segment (start 44.075 35) (end 44.075 35.45) (width 0.2) (layer "F.Cu") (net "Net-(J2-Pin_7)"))
 (segment (start 44.15 36.1) (end 43.75 36.5) (width 0.2) (layer "F.Cu") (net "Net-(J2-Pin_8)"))
 (segment (start 43.75 36.5) (end 41.28 36.5) (width 0.2) (layer "F.Cu") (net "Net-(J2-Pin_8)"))
 (segment (start 41.28 36.5) (end 39.78 38) (width 0.2) (layer "F.Cu") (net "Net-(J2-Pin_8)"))
 (segment (start 45.25 36.1) (end 44.15 36.1) (width 0.2) (layer "F.Cu") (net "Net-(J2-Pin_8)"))
 (segment (start 45.345 35) (end 45.345 36.005) (width 0.2) (layer "F.Cu") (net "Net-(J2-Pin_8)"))
 (segment (start 45.345 36.005) (end 45.25 36.1) (width 0.2) (layer "F.Cu") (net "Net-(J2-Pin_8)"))
 (segment (start 46.58 35.035) (end 46.58 35.714314) (width 0.2) (layer "F.Cu") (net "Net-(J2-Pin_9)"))
 (segment (start 44.41 36.5) (end 42.91 38) (width 0.2) (layer "F.Cu") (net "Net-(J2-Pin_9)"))
 (segment (start 46.58 35.714314) (end 45.794315 36.5) (width 0.2) (layer "F.Cu") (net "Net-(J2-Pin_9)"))
 (segment (start 42.91 38) (end 42.32 38) (width 0.2) (layer "F.Cu") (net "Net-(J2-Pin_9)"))
 (segment (start 45.794315 36.5) (end 44.41 36.5) (width 0.2) (layer "F.Cu") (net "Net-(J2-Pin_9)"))
 (segment (start 46.615 35) (end 46.58 35.035) (width 0.2) (layer "F.Cu") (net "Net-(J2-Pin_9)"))
 (segment (start 46.5 36.5) (end 45 38) (width 0.2) (layer "F.Cu") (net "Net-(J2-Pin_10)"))
 (segment (start 45 38) (end 44.86 38) (width 0.2) (layer "F.Cu") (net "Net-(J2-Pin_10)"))
 (segment (start 47.85 36.15) (end 47.5 36.5) (width 0.2) (layer "F.Cu") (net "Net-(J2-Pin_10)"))
 (segment (start 47.885 35) (end 47.85 35.035) (width 0.2) (layer "F.Cu") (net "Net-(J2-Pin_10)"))
 (segment (start 47.5 36.5) (end 46.5 36.5) (width 0.2) (layer "F.Cu") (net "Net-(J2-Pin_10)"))
 (segment (start 47.85 35.035) (end 47.85 36.15) (width 0.2) (layer "F.Cu") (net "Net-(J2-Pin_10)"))
 (segment (start 49.155 35) (end 49.12 35.035) (width 0.2) (layer "F.Cu") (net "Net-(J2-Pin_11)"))
 (segment (start 49.12 36.28) (end 47.4 38) (width 0.2) (layer "F.Cu") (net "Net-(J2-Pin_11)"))
 (segment (start 49.12 35.035) (end 49.12 36.28) (width 0.2) (layer "F.Cu") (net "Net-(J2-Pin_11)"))
 (segment (start 50.425 35) (end 50.39 35.035) (width 0.2) (layer "F.Cu") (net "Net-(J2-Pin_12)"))
 (segment (start 50.39 37.55) (end 49.94 38) (width 0.2) (layer "F.Cu") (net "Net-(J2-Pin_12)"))
 (segment (start 50.39 35.035) (end 50.39 37.55) (width 0.2) (layer "F.Cu") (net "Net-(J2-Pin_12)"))
 (segment (start 51.695 35) (end 51.66 35.035) (width 0.2) (layer "F.Cu") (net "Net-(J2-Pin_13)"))
 (segment (start 51.66 37.18) (end 52.48 38) (width 0.2) (layer "F.Cu") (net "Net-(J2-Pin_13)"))
 (segment (start 51.66 35.035) (end 51.66 37.18) (width 0.2) (layer "F.Cu") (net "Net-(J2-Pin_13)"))
 (segment (start 30 22.38) (end 29.62 22) (width 0.2) (layer "F.Cu") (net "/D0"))
 (segment (start 30 26) (end 30 22.38) (width 0.2) (layer "F.Cu") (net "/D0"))
 (segment (start 51.695 25.95) (end 51.695 25.5) (width 0.2) (layer "F.Cu") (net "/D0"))
 (segment (start 31.27 22.89) (end 32.16 22) (width 0.2) (layer "F.Cu") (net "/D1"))
 (segment (start 31.27 26) (end 31.27 22.89) (width 0.2) (layer "F.Cu") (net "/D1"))
 (segment (start 50.425 25.95) (end 50.425 25.5) (width 0.2) (layer "F.Cu") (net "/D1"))
 (segment (start 32.54 24.16) (end 34.7 22) (width 0.2) (layer "F.Cu") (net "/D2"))
 (segment (start 32.54 26) (end 32.54 24.16) (width 0.2) (layer "F.Cu") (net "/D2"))
 (segment (start 49.155 25.95) (end 49.155 25.5) (width 0.2) (layer "F.Cu") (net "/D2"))
 (segment (start 47.885 25.95) (end 47.885 25.5) (width 0.2) (layer "F.Cu") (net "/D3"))
 (segment (start 33.81 26) (end 33.81 24.44) (width 0.2) (layer "F.Cu") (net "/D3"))
 (segment (start 33.81 24.44) (end 34.25 24) (width 0.2) (layer "F.Cu") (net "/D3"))
 (segment (start 34.25 24) (end 35.24 24) (width 0.2) (layer "F.Cu") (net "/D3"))
 (segment (start 35.24 24) (end 37.24 22) (width 0.2) (layer "F.Cu") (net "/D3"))
 (segment (start 38 23.5) (end 39.5 22) (width 0.2) (layer "F.Cu") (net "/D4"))
 (segment (start 35.08 26) (end 35.08 24.92) (width 0.2) (layer "F.Cu") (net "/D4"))
 (segment (start 46.615 26.185) (end 46.615 25.5) (width 0.2) (layer "F.Cu") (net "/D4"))
 (segment (start 36.5 23.5) (end 38 23.5) (width 0.2) (layer "F.Cu") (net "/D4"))
 (segment (start 39.5 22) (end 39.78 22) (width 0.2) (layer "F.Cu") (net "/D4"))
 (segment (start 35.08 24.92) (end 36.5 23.5) (width 0.2) (layer "F.Cu") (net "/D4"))
 (segment (start 40.787157 23.532843) (end 38.532843 23.532843) (width 0.2) (layer "F.Cu") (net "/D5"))
 (segment (start 38.532843 23.532843) (end 38.065686 24) (width 0.2) (layer "F.Cu") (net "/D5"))
 (segment (start 36.862501 24) (end 36.35 24.512501) (width 0.2) (layer "F.Cu") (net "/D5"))
 (segment (start 38.065686 24) (end 36.862501 24) (width 0.2) (layer "F.Cu") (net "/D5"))
 (segment (start 36.35 24.512501) (end 36.35 25.445) (width 0.2) (layer "F.Cu") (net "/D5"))
 (segment (start 42.32 22) (end 40.787157 23.532843) (width 0.2) (layer "F.Cu") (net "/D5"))
 (segment (start 44.075 25.5) (end 44.075 24) (width 0.2) (layer "F.Cu") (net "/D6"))
 (segment (start 42.205 24.295) (end 42.205 26.48) (width 0.2) (layer "F.Cu") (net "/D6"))
 (segment (start 41.1 26.6) (end 40.5 26) (width 0.2) (layer "F.Cu") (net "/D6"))
 (segment (start 44.075 24) (end 44.075 22.785) (width 0.2) (layer "F.Cu") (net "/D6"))
 (segment (start 40.5 24.5) (end 40 24) (width 0.2) (layer "F.Cu") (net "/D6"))
 (segment (start 40.5 26) (end 40.5 24.5) (width 0.2) (layer "F.Cu") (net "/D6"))
 (segment (start 44.075 24) (end 42.5 24) (width 0.2) (layer "F.Cu") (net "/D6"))
 (segment (start 42.5 24) (end 42.205 24.295) (width 0.2) (layer "F.Cu") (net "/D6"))
 (segment (start 40 24) (end 38.632501 24) (width 0.2) (layer "F.Cu") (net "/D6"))
 (segment (start 37.62 25.012501) (end 37.62 26) (width 0.2) (layer "F.Cu") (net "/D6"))
 (segment (start 38.632501 24) (end 37.62 25.012501) (width 0.2) (layer "F.Cu") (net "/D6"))
 (segment (start 42.085 26.6) (end 41.1 26.6) (width 0.2) (layer "F.Cu") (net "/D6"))
 (segment (start 42.205 26.48) (end 42.085 26.6) (width 0.2) (layer "F.Cu") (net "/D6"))
 (segment (start 44.075 22.785) (end 44.86 22) (width 0.2) (layer "F.Cu") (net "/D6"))
 (segment (start 47.4 23.1) (end 46.75 23.75) (width 0.2) (layer "F.Cu") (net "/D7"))
 (segment (start 44.745 26.505) (end 44.65 26.6) (width 0.2) (layer "F.Cu") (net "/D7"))
 (segment (start 44.745 24.255) (end 44.745 26.505) (width 0.2) (layer "F.Cu") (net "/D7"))
 (segment (start 47.4 22) (end 47.4 23.1) (width 0.2) (layer "F.Cu") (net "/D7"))
 (segment (start 44.65 26.6) (end 43.455 26.6) (width 0.2) (layer "F.Cu") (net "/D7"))
 (segment (start 45.25 23.75) (end 44.745 24.255) (width 0.2) (layer "F.Cu") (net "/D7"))
 (segment (start 43.455 26.6) (end 42.805 25.95) (width 0.2) (layer "F.Cu") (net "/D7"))
 (segment (start 46.75 23.75) (end 45.25 23.75) (width 0.2) (layer "F.Cu") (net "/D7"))
 (segment (start 42.805 25.95) (end 42.805 25.5) (width 0.2) (layer "F.Cu") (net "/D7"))
 (segment (start 23.5 23.5) (end 24.75 24.75) (width 0.5) (layer "F.Cu") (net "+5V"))
 (segment (start 22.25 23.5) (end 23.5 23.5) (width 0.5) (layer "F.Cu") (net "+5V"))
 (segment (start 22 23.25) (end 22.25 23.5) (width 0.5) (layer "F.Cu") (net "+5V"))
 (segment (start 22 22) (end 22 23.25) (width 0.5) (layer "F.Cu") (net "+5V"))
 (segment (start 28.6 26.4) (end 26.6 26.4) (width 0.2) (layer "F.Cu") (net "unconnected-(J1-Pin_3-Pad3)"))
 (segment (start 27.08 22) (end 27.08 23.33) (width 0.2) (layer "F.Cu") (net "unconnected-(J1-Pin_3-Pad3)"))
 (segment (start 28.9 25.15) (end 28.9 26.1) (width 0.2) (layer "F.Cu") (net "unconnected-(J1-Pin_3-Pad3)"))
 (segment (start 27.08 23.33) (end 28.9 25.15) (width 0.2) (layer "F.Cu") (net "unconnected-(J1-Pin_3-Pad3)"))
 (segment (start 28.9 26.1) (end 28.6 26.4) (width 0.2) (layer "F.Cu") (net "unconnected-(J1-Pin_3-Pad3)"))
 (segment (start 60.5 23.75) (end 60 24.25) (width 0.2) (layer "F.Cu") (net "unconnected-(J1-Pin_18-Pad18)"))
 (segment (start 64 23.75) (end 60.5 23.75) (width 0.2) (layer "F.Cu") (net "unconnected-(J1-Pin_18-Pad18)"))
 (segment (start 65.18 22) (end 65.18 22.57) (width 0.2) (layer "F.Cu") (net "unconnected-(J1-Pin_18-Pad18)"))
 (segment (start 65.18 22.57) (end 64 23.75) (width 0.2) (layer "F.Cu") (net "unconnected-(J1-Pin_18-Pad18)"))
 (segment (start 60 24.25) (end 60 26) (width 0.2) (layer "F.Cu") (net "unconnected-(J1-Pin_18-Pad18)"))
 (segment (start 70.26 22) (end 70.26 23.74) (width 0.2) (layer "F.Cu") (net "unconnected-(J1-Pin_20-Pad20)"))
 (segment (start 68.25 25.75) (end 68.25 26.5) (width 0.2) (layer "F.Cu") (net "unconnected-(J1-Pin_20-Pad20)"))
 (segment (start 70.26 23.74) (end 68.25 25.75) (width 0.2) (layer "F.Cu") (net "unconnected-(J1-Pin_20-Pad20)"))
 (segment (start 30 34) (end 29.455 33.455) (width 0.2) (layer "F.Cu") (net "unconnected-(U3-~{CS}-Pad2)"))
 (segment (start 29.455 33.455) (end 29.455 31.75) (width 0.2) (layer "F.Cu") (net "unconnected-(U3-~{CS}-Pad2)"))
 (segment (start 31.325 33.425) (end 30.75 34) (width 0.2) (layer "F.Cu") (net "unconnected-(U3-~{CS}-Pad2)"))
 (segment (start 31.325 32.425) (end 31.325 33.425) (width 0.2) (layer "F.Cu") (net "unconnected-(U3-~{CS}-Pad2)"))
 (segment (start 30.75 34) (end 30 34) (width 0.2) (layer "F.Cu") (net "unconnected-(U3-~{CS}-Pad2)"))
 (segment (start 39.5 34) (end 40.25 33.25) (width 0.2) (layer "F.Cu") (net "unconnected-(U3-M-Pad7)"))
 (segment (start 37.675 32.425) (end 37.675 33.412499) (width 0.2) (layer "F.Cu") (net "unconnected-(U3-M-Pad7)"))
 (segment (start 37.675 33.412499) (end 38.262501 34) (width 0.2) (layer "F.Cu") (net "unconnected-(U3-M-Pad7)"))
 (segment (start 38.262501 34) (end 39.5 34) (width 0.2) (layer "F.Cu") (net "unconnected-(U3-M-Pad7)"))
 (segment (start 40.075 32.425) (end 41 31.5) (width 0.2) (layer "F.Cu") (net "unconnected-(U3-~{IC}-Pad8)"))
 (segment (start 38.945 32.425) (end 40.075 32.425) (width 0.2) (layer "F.Cu") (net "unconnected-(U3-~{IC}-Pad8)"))
 (segment (start 37.005 34.005) (end 37.005 31.755) (width 0.2) (layer "F.Cu") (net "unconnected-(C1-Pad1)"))
 (segment (start 37.65 34.65) (end 37.005 34.005) (width 0.2) (layer "F.Cu") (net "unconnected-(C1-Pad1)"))
 (segment (start 37.65 35.25) (end 37.65 34.65) (width 0.2) (layer "F.Cu") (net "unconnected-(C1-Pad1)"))
 (segment (start 37.65 35.25) (end 39.75 35.25) (width 0.5) (layer "F.Cu") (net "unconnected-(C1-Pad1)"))
 (segment (start 39.75 34.527818) (end 40.527818 33.75) (width 0.5) (layer "F.Cu") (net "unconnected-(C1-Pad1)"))
 (segment (start 39.75 35.25) (end 39.75 34.527818) (width 0.5) (layer "F.Cu") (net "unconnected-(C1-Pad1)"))
 (via (at 39.75 35.25) (size 0.6) (drill 0.3) (layers "F.Cu" "B.Cu") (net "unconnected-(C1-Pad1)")))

